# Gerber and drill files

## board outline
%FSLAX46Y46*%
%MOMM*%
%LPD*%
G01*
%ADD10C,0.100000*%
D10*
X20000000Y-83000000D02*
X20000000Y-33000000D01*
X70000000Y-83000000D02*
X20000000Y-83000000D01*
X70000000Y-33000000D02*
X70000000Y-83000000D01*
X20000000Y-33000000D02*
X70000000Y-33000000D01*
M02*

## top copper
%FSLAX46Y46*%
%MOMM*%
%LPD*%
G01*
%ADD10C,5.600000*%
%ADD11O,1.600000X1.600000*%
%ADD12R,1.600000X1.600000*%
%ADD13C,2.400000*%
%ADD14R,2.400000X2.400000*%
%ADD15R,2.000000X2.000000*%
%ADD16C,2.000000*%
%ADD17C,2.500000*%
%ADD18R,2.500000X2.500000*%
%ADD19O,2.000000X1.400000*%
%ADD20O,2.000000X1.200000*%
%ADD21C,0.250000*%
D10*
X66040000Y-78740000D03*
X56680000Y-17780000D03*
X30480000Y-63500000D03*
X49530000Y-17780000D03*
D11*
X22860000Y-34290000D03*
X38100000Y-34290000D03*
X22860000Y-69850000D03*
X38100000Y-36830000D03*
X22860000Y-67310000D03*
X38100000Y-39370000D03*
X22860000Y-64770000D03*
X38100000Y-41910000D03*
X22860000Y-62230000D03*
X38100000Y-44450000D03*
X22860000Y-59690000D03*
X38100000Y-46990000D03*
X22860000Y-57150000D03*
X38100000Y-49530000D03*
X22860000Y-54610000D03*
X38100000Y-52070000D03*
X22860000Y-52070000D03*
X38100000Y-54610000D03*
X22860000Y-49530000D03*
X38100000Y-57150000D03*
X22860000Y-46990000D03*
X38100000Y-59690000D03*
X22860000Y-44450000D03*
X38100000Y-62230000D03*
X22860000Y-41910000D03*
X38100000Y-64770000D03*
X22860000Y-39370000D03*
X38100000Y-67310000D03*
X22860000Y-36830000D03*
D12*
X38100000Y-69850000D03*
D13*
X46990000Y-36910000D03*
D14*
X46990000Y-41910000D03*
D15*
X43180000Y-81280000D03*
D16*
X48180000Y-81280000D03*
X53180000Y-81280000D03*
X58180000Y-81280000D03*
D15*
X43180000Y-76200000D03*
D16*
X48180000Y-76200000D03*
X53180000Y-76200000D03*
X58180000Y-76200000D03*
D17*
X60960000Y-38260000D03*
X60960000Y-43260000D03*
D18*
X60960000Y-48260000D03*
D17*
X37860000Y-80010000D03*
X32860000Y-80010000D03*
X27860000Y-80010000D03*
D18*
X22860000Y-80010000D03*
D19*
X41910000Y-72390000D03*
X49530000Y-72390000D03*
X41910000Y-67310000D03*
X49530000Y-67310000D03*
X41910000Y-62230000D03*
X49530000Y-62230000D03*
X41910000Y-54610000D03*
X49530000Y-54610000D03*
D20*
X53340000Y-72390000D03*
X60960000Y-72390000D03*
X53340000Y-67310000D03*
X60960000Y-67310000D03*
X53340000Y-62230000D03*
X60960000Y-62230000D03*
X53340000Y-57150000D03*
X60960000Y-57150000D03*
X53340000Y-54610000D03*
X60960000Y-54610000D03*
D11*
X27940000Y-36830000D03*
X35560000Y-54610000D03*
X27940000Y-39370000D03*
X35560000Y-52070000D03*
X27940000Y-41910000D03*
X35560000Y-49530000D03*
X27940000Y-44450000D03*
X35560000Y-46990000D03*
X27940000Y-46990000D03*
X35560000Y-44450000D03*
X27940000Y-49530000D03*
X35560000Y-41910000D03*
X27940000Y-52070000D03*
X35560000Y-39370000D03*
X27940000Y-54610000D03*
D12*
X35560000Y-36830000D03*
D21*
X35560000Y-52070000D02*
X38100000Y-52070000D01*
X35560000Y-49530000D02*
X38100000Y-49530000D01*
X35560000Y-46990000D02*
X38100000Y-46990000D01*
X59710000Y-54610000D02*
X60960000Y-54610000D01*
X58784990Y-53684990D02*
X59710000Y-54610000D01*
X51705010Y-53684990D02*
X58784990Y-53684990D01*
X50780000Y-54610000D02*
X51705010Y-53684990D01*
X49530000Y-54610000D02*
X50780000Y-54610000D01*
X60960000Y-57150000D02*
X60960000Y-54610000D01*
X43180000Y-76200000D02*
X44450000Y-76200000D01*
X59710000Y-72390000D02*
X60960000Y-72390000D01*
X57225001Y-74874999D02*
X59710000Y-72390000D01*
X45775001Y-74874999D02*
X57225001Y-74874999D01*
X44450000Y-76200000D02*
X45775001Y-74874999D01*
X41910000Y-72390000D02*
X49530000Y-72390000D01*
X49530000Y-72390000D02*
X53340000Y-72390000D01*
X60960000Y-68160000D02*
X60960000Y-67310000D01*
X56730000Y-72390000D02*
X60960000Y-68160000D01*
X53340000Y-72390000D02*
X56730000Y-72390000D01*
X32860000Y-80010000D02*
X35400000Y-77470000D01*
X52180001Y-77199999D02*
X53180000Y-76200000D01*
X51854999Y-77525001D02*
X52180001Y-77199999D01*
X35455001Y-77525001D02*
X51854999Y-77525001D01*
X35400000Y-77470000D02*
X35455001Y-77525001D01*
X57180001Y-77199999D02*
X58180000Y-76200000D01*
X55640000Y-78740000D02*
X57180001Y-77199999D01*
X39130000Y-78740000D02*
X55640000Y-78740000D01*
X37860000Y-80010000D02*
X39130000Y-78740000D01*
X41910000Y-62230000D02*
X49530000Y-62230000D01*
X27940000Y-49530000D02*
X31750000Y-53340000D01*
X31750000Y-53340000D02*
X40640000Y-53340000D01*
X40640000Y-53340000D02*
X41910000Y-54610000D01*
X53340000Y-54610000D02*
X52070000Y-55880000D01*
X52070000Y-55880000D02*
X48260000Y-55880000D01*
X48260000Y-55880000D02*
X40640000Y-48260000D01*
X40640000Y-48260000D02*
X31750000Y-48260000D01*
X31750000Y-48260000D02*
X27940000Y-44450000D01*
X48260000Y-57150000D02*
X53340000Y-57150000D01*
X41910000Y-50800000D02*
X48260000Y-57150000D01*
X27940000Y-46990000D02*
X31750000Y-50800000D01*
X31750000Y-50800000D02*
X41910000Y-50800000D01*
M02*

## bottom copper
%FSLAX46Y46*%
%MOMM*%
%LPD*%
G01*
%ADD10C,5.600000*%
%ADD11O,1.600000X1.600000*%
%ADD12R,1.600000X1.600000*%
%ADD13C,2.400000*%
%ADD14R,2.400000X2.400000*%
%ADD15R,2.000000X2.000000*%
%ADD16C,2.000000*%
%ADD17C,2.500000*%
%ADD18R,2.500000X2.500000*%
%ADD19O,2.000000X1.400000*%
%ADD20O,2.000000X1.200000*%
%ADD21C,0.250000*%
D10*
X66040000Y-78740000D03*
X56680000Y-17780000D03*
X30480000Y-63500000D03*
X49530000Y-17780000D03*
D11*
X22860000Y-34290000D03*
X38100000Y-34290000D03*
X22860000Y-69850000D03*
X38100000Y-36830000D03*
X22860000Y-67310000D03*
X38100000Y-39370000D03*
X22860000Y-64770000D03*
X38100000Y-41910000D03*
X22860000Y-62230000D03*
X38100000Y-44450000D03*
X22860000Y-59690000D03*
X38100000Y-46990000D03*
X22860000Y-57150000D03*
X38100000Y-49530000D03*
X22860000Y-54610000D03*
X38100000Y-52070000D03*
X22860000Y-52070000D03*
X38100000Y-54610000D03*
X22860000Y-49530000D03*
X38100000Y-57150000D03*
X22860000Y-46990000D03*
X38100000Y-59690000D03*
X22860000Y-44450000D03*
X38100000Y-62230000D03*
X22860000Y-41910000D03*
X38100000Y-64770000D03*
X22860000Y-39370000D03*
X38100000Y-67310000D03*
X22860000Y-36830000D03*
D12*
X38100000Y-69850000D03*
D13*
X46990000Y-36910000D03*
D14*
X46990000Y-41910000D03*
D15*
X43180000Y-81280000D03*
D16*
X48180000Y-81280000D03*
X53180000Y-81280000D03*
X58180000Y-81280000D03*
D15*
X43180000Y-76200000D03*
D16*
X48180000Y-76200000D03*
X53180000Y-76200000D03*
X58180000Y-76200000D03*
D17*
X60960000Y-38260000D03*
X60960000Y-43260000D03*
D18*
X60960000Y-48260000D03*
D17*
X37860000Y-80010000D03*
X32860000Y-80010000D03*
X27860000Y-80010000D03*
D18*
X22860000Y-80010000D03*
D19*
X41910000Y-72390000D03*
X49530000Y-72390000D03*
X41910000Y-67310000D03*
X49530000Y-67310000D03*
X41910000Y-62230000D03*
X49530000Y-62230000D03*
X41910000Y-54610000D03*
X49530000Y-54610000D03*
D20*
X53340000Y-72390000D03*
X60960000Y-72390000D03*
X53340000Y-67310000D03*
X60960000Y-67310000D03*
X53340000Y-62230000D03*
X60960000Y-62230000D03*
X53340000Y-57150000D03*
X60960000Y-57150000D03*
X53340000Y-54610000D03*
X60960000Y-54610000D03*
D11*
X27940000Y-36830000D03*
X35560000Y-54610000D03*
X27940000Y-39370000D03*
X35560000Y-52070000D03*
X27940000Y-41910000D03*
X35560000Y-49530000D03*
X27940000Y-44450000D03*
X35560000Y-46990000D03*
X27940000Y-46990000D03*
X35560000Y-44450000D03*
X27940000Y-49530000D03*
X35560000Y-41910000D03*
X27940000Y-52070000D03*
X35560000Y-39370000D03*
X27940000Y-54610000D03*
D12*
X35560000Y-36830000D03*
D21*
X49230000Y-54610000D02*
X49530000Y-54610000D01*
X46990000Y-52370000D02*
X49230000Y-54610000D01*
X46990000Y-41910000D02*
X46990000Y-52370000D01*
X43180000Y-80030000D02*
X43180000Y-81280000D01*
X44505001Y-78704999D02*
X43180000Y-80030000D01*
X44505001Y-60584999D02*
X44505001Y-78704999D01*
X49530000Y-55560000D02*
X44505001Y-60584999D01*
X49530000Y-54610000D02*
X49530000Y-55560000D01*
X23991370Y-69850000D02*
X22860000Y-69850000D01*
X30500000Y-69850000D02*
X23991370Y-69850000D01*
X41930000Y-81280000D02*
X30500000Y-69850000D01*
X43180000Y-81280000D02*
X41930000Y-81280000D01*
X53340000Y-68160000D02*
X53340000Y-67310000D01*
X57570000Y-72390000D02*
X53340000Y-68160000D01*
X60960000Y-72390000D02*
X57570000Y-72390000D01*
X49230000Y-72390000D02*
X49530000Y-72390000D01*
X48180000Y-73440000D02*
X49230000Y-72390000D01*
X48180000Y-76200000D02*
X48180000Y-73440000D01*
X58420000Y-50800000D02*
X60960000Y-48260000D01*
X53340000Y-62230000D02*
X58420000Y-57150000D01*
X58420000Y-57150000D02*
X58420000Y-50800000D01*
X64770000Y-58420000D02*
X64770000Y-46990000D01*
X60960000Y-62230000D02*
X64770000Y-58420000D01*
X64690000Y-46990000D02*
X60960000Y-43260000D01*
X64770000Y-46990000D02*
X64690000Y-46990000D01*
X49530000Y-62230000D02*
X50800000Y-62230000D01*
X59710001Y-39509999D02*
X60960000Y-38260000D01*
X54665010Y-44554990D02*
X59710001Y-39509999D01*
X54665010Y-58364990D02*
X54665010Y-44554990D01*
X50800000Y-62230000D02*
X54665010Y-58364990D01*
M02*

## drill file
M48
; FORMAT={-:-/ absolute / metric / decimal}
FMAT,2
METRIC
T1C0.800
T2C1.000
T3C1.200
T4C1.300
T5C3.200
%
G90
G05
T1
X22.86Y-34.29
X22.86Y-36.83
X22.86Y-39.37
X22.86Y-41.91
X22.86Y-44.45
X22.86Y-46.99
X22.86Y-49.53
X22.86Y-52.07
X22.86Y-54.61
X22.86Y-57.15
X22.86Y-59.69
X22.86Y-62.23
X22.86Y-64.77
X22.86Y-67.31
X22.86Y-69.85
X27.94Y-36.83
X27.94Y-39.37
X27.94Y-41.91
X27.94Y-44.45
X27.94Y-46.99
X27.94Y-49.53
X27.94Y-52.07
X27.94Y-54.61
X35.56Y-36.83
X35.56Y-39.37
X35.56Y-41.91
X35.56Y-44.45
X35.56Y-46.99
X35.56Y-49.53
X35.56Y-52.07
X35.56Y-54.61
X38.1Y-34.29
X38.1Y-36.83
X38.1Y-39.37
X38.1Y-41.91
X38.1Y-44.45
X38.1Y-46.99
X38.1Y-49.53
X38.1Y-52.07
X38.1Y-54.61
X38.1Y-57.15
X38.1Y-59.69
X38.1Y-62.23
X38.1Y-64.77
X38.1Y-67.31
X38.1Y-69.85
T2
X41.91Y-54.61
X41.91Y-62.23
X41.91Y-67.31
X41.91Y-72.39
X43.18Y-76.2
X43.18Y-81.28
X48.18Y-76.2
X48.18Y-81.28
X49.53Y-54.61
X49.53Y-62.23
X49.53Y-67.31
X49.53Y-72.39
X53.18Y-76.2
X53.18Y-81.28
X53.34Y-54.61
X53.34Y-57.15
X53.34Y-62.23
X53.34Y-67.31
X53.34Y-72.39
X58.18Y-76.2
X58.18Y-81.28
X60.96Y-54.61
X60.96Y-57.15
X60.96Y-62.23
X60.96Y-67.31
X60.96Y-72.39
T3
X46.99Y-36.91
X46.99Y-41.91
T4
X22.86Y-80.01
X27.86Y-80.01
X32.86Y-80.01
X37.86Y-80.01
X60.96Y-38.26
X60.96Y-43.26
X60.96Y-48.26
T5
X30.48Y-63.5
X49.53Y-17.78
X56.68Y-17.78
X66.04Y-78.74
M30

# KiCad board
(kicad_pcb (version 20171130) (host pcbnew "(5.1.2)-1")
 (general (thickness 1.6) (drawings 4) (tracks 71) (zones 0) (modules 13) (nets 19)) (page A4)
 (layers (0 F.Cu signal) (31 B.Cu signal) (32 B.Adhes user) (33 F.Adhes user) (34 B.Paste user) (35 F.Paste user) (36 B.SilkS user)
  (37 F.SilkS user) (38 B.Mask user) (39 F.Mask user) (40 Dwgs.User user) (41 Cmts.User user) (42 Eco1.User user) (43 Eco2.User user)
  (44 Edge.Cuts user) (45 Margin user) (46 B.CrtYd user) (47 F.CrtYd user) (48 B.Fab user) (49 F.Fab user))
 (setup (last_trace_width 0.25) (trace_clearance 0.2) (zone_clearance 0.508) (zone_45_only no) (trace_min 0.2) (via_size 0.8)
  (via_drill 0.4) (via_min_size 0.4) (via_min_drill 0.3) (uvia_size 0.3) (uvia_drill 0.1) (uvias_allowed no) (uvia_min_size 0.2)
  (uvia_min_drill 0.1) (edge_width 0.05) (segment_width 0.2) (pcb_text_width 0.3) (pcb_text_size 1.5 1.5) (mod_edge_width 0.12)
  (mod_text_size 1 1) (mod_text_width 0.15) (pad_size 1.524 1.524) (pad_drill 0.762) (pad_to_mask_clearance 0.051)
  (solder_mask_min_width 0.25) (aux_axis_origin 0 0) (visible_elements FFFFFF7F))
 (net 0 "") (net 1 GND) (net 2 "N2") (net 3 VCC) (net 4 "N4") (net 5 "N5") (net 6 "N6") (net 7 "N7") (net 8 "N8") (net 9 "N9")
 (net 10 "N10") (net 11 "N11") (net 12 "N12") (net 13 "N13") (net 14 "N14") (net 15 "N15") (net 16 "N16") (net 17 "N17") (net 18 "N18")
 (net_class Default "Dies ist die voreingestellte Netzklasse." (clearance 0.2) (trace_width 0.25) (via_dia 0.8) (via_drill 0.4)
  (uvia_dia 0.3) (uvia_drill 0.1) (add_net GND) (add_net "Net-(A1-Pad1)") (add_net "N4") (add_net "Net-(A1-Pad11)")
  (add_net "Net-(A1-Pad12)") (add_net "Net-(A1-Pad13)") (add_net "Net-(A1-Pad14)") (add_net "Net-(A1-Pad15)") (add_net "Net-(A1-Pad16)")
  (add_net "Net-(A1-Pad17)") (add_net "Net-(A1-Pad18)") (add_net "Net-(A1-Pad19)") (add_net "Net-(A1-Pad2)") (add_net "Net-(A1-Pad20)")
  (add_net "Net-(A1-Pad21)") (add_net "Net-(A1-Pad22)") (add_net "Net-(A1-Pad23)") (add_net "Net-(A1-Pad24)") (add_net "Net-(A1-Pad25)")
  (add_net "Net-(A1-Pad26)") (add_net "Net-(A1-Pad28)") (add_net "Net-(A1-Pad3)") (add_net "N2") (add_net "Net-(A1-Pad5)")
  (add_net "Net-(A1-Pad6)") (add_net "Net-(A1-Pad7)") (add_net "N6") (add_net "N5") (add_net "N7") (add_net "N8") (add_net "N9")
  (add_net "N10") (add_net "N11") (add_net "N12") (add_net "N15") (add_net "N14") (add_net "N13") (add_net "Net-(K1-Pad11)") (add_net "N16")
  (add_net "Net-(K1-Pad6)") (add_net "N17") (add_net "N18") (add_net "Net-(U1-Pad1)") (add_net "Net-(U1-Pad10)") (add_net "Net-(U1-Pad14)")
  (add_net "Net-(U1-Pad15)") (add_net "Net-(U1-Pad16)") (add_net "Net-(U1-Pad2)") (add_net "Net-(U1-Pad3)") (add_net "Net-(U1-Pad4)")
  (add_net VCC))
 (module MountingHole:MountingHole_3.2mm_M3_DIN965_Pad (layer F.Cu) (at 66.04 78.74)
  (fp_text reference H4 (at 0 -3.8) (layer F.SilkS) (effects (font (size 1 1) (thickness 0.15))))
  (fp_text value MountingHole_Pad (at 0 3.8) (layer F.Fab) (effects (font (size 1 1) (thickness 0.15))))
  (pad 1 thru_hole circle (at 0 0) (size 5.6 5.6) (drill 3.2) (layers *.Cu *.Mask) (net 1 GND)))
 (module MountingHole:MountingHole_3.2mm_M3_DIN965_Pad (layer F.Cu) (at 56.68 17.78)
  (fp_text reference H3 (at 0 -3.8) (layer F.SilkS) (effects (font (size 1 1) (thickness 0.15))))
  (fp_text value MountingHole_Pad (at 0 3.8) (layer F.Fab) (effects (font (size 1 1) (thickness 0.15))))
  (pad 1 thru_hole circle (at 0 0) (size 5.6 5.6) (drill 3.2) (layers *.Cu *.Mask) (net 1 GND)))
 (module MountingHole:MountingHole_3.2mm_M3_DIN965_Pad (layer F.Cu) (at 30.48 63.5)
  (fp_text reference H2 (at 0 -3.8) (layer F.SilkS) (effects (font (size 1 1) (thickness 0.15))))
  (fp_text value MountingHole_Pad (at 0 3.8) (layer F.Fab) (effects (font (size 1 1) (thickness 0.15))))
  (pad 1 thru_hole circle (at 0 0) (size 5.6 5.6) (drill 3.2) (layers *.Cu *.Mask) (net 1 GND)))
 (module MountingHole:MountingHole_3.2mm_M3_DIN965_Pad (layer F.Cu) (at 49.53 17.78)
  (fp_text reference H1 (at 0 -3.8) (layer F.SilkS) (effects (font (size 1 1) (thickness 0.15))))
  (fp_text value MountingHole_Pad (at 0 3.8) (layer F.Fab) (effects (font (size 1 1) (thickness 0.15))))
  (pad 1 thru_hole circle (at 0 0) (size 5.6 5.6) (drill 3.2) (layers *.Cu *.Mask) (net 1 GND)))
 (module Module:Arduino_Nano (layer F.Cu) (at 38.1 69.85 180)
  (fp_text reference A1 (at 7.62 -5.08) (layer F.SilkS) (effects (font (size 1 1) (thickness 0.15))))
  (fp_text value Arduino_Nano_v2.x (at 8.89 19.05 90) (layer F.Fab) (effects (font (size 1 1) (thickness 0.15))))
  (pad 16 thru_hole oval (at 15.24 35.56 180) (size 1.6 1.6) (drill 0.8) (layers *.Cu *.Mask))
  (pad 15 thru_hole oval (at 0 35.56 180) (size 1.6 1.6) (drill 0.8) (layers *.Cu *.Mask))
  (pad 30 thru_hole oval (at 15.24 0 180) (size 1.6 1.6) (drill 0.8) (layers *.Cu *.Mask) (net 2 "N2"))
  (pad 14 thru_hole oval (at 0 33.02 180) (size 1.6 1.6) (drill 0.8) (layers *.Cu *.Mask))
  (pad 29 thru_hole oval (at 15.24 2.54 180) (size 1.6 1.6) (drill 0.8) (layers *.Cu *.Mask) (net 1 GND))
  (pad 13 thru_hole oval (at 0 30.48 180) (size 1.6 1.6) (drill 0.8) (layers *.Cu *.Mask))
  (pad 28 thru_hole oval (at 15.24 5.08 180) (size 1.6 1.6) (drill 0.8) (layers *.Cu *.Mask))
  (pad 12 thru_hole oval (at 0 27.94 180) (size 1.6 1.6) (drill 0.8) (layers *.Cu *.Mask))
  (pad 27 thru_hole oval (at 15.24 7.62 180) (size 1.6 1.6) (drill 0.8) (layers *.Cu *.Mask) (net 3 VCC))
  (pad 11 thru_hole oval (at 0 25.4 180) (size 1.6 1.6) (drill 0.8) (layers *.Cu *.Mask))
  (pad 26 thru_hole oval (at 15.24 10.16 180) (size 1.6 1.6) (drill 0.8) (layers *.Cu *.Mask))
  (pad 10 thru_hole oval (at 0 22.86 180) (size 1.6 1.6) (drill 0.8) (layers *.Cu *.Mask) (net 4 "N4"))
  (pad 25 thru_hole oval (at 15.24 12.7 180) (size 1.6 1.6) (drill 0.8) (layers *.Cu *.Mask))
  (pad 9 thru_hole oval (at 0 20.32 180) (size 1.6 1.6) (drill 0.8) (layers *.Cu *.Mask) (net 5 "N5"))
  (pad 24 thru_hole oval (at 15.24 15.24 180) (size 1.6 1.6) (drill 0.8) (layers *.Cu *.Mask))
  (pad 8 thru_hole oval (at 0 17.78 180) (size 1.6 1.6) (drill 0.8) (layers *.Cu *.Mask) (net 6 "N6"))
  (pad 23 thru_hole oval (at 15.24 17.78 180) (size 1.6 1.6) (drill 0.8) (layers *.Cu *.Mask))
  (pad 7 thru_hole oval (at 0 15.24 180) (size 1.6 1.6) (drill 0.8) (layers *.Cu *.Mask))
  (pad 22 thru_hole oval (at 15.24 20.32 180) (size 1.6 1.6) (drill 0.8) (layers *.Cu *.Mask))
  (pad 6 thru_hole oval (at 0 12.7 180) (size 1.6 1.6) (drill 0.8) (layers *.Cu *.Mask))
  (pad 21 thru_hole oval (at 15.24 22.86 180) (size 1.6 1.6) (drill 0.8) (layers *.Cu *.Mask))
  (pad 5 thru_hole oval (at 0 10.16 180) (size 1.6 1.6) (drill 0.8) (layers *.Cu *.Mask))
  (pad 20 thru_hole oval (at 15.24 25.4 180) (size 1.6 1.6) (drill 0.8) (layers *.Cu *.Mask))
  (pad 4 thru_hole oval (at 0 7.62 180) (size 1.6 1.6) (drill 0.8) (layers *.Cu *.Mask) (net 1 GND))
  (pad 19 thru_hole oval (at 15.24 27.94 180) (size 1.6 1.6) (drill 0.8) (layers *.Cu *.Mask))
  (pad 3 thru_hole oval (at 0 5.08 180) (size 1.6 1.6) (drill 0.8) (layers *.Cu *.Mask))
  (pad 18 thru_hole oval (at 15.24 30.48 180) (size 1.6 1.6) (drill 0.8) (layers *.Cu *.Mask))
  (pad 2 thru_hole oval (at 0 2.54 180) (size 1.6 1.6) (drill 0.8) (layers *.Cu *.Mask))
  (pad 17 thru_hole oval (at 15.24 33.02 180) (size 1.6 1.6) (drill 0.8) (layers *.Cu *.Mask))
  (pad 1 thru_hole rect (at 0 0 180) (size 1.6 1.6) (drill 0.8) (layers *.Cu *.Mask)))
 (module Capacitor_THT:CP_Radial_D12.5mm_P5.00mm (layer F.Cu) (at 46.99 41.91 90)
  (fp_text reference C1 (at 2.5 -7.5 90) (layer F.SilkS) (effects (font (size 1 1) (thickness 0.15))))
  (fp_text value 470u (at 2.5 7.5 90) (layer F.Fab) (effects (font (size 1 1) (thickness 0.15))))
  (pad 2 thru_hole circle (at 5 0 90) (size 2.4 2.4) (drill 1.2) (layers *.Cu *.Mask) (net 1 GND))
  (pad 1 thru_hole rect (at 0 0 90) (size 2.4 2.4) (drill 1.2) (layers *.Cu *.Mask) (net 3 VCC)))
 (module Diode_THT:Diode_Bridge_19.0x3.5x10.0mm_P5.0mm (layer F.Cu) (at 43.18 81.28)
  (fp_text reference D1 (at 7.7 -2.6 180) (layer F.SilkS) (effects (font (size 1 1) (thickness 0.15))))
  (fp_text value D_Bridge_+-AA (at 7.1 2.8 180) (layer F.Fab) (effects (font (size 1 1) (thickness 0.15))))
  (pad 1 thru_hole rect (at 0 0) (size 2 2) (drill 1) (layers *.Cu *.Mask) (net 2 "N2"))
  (pad 2 thru_hole circle (at 5 0) (size 2 2) (drill 1) (layers *.Cu *.Mask) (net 1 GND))
  (pad 3 thru_hole circle (at 10 0) (size 2 2) (drill 1) (layers *.Cu *.Mask) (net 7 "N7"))
  (pad 4 thru_hole circle (at 15 0) (size 2 2) (drill 1) (layers *.Cu *.Mask) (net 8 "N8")))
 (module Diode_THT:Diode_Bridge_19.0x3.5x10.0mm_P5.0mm (layer F.Cu) (at 43.18 76.2)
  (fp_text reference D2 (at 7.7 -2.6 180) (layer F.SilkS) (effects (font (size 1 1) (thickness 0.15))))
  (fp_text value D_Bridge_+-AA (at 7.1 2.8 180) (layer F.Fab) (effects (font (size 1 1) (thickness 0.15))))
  (pad 1 thru_hole rect (at 0 0) (size 2 2) (drill 1) (layers *.Cu *.Mask) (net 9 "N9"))
  (pad 2 thru_hole circle (at 5 0) (size 2 2) (drill 1) (layers *.Cu *.Mask) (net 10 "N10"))
  (pad 3 thru_hole circle (at 10 0) (size 2 2) (drill 1) (layers *.Cu *.Mask) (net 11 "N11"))
  (pad 4 thru_hole circle (at 15 0) (size 2 2) (drill 1) (layers *.Cu *.Mask) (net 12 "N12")))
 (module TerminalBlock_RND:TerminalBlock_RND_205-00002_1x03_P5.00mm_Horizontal (layer F.Cu) (at 60.96 48.26 90)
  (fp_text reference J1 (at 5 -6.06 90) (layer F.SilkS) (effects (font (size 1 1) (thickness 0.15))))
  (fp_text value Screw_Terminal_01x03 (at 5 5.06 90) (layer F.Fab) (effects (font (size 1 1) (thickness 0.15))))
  (pad 3 thru_hole circle (at 10 0 90) (size 2.5 2.5) (drill 1.3) (layers *.Cu *.Mask) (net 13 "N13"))
  (pad 2 thru_hole circle (at 5 0 90) (size 2.5 2.5) (drill 1.3) (layers *.Cu *.Mask) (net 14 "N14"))
  (pad 1 thru_hole rect (at 0 0 90) (size 2.5 2.5) (drill 1.3) (layers *.Cu *.Mask) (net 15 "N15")))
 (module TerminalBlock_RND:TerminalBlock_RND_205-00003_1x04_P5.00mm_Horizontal (layer F.Cu) (at 22.86 80.01)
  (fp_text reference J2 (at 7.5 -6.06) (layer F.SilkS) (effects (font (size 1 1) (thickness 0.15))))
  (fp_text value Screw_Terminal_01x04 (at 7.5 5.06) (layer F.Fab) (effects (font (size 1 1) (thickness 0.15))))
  (pad 4 thru_hole circle (at 15 0) (size 2.5 2.5) (drill 1.3) (layers *.Cu *.Mask) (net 12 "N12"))
  (pad 3 thru_hole circle (at 10 0) (size 2.5 2.5) (drill 1.3) (layers *.Cu *.Mask) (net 11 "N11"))
  (pad 2 thru_hole circle (at 5 0) (size 2.5 2.5) (drill 1.3) (layers *.Cu *.Mask) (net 8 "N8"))
  (pad 1 thru_hole rect (at 0 0) (size 2.5 2.5) (drill 1.3) (layers *.Cu *.Mask) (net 7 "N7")))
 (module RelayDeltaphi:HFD (layer F.Cu) (at 45.72 63.5 270)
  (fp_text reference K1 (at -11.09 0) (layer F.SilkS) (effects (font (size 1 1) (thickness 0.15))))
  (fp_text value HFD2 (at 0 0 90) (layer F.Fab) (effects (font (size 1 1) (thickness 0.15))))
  (pad 9 thru_hole oval (at 8.89 3.81 270) (size 1.4 2) (drill 1) (layers *.Cu *.Mask) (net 10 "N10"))
  (pad 8 thru_hole oval (at 8.89 -3.81 270) (size 1.4 2) (drill 1) (layers *.Cu *.Mask) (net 10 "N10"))
  (pad 11 thru_hole oval (at 3.81 3.81 270) (size 1.4 2) (drill 1) (layers *.Cu *.Mask))
  (pad 6 thru_hole oval (at 3.81 -3.81 270) (size 1.4 2) (drill 1) (layers *.Cu *.Mask))
  (pad 13 thru_hole oval (at -1.27 3.81 270) (size 1.4 2) (drill 1) (layers *.Cu *.Mask) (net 13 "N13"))
  (pad 4 thru_hole oval (at -1.27 -3.81 270) (size 1.4 2) (drill 1) (layers *.Cu *.Mask) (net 13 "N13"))
  (pad 16 thru_hole oval (at -8.89 3.81 270) (size 1.4 2) (drill 1) (layers *.Cu *.Mask) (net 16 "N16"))
  (pad 1 thru_hole oval (at -8.89 -3.81 270) (size 1.4 2) (drill 1) (layers *.Cu *.Mask) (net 3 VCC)))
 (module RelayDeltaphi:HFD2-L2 (layer F.Cu) (at 57.15 63.5 270)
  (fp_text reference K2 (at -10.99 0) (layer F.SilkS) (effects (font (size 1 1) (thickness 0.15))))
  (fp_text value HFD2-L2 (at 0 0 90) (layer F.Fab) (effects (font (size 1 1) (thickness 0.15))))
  (pad 9 thru_hole oval (at 8.89 3.81 270) (size 1.2 2) (drill 1) (layers *.Cu *.Mask) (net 10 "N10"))
  (pad 8 thru_hole oval (at 8.89 -3.81 270) (size 1.2 2) (drill 1) (layers *.Cu *.Mask) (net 9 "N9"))
  (pad 11 thru_hole oval (at 3.81 3.81 270) (size 1.2 2) (drill 1) (layers *.Cu *.Mask) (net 9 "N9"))
  (pad 6 thru_hole oval (at 3.81 -3.81 270) (size 1.2 2) (drill 1) (layers *.Cu *.Mask) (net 10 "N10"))
  (pad 13 thru_hole oval (at -1.27 3.81 270) (size 1.2 2) (drill 1) (layers *.Cu *.Mask) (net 15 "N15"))
  (pad 4 thru_hole oval (at -1.27 -3.81 270) (size 1.2 2) (drill 1) (layers *.Cu *.Mask) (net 14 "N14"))
  (pad 15 thru_hole oval (at -6.35 3.81 270) (size 1.2 2) (drill 1) (layers *.Cu *.Mask) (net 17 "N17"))
  (pad 2 thru_hole oval (at -6.35 -3.81 270) (size 1.2 2) (drill 1) (layers *.Cu *.Mask) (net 3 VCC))
  (pad 16 thru_hole oval (at -8.89 3.81 270) (size 1.2 2) (drill 1) (layers *.Cu *.Mask) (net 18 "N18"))
  (pad 1 thru_hole oval (at -8.89 -3.81 270) (size 1.2 2) (drill 1) (layers *.Cu *.Mask) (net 3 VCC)))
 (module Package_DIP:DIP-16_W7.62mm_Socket (layer B.Cu) (at 35.56 36.83 180)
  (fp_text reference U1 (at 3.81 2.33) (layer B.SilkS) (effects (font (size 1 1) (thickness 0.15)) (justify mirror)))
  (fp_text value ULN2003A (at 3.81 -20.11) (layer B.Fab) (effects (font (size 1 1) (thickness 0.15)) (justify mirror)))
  (pad 16 thru_hole oval (at 7.62 0 180) (size 1.6 1.6) (drill 0.8) (layers *.Cu *.Mask))
  (pad 8 thru_hole oval (at 0 -17.78 180) (size 1.6 1.6) (drill 0.8) (layers *.Cu *.Mask) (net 1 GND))
  (pad 15 thru_hole oval (at 7.62 -2.54 180) (size 1.6 1.6) (drill 0.8) (layers *.Cu *.Mask))
  (pad 7 thru_hole oval (at 0 -15.24 180) (size 1.6 1.6) (drill 0.8) (layers *.Cu *.Mask) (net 6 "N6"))
  (pad 14 thru_hole oval (at 7.62 -5.08 180) (size 1.6 1.6) (drill 0.8) (layers *.Cu *.Mask))
  (pad 6 thru_hole oval (at 0 -12.7 180) (size 1.6 1.6) (drill 0.8) (layers *.Cu *.Mask) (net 5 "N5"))
  (pad 13 thru_hole oval (at 7.62 -7.62 180) (size 1.6 1.6) (drill 0.8) (layers *.Cu *.Mask) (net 18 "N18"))
  (pad 5 thru_hole oval (at 0 -10.16 180) (size 1.6 1.6) (drill 0.8) (layers *.Cu *.Mask) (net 4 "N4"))
  (pad 12 thru_hole oval (at 7.62 -10.16 180) (size 1.6 1.6) (drill 0.8) (layers *.Cu *.Mask) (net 17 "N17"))
  (pad 4 thru_hole oval (at 0 -7.62 180) (size 1.6 1.6) (drill 0.8) (layers *.Cu *.Mask))
  (pad 11 thru_hole oval (at 7.62 -12.7 180) (size 1.6 1.6) (drill 0.8) (layers *.Cu *.Mask) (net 16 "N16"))
  (pad 3 thru_hole oval (at 0 -5.08 180) (size 1.6 1.6) (drill 0.8) (layers *.Cu *.Mask))
  (pad 10 thru_hole oval (at 7.62 -15.24 180) (size 1.6 1.6) (drill 0.8) (layers *.Cu *.Mask))
  (pad 2 thru_hole oval (at 0 -2.54 180) (size 1.6 1.6) (drill 0.8) (layers *.Cu *.Mask))
  (pad 9 thru_hole oval (at 7.62 -17.78 180) (size 1.6 1.6) (drill 0.8) (layers *.Cu *.Mask) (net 1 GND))
  (pad 1 thru_hole rect (at 0 0 180) (size 1.6 1.6) (drill 0.8) (layers *.Cu *.Mask)))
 (gr_line (start 20 83) (end 20 33) (layer Edge.Cuts) (width 0.1))
 (gr_line (start 70 83) (end 20 83) (layer Edge.Cuts) (width 0.1))
 (gr_line (start 70 33) (end 70 83) (layer Edge.Cuts) (width 0.1))
 (gr_line (start 20 33) (end 70 33) (layer Edge.Cuts) (width 0.1))
 (segment (start 35.56 52.07) (end 38.1 52.07) (width 0.25) (layer F.Cu) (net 6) (status 30))
 (segment (start 35.56 49.53) (end 38.1 49.53) (width 0.25) (layer F.Cu) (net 5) (status 30))
 (segment (start 35.56 46.99) (end 38.1 46.99) (width 0.25) (layer F.Cu) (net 4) (status 30))
 (segment (start 59.71 54.61) (end 60.96 54.61) (width 0.25) (layer F.Cu) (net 3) (status 20))
 (segment (start 58.78499 53.68499) (end 59.71 54.61) (width 0.25) (layer F.Cu) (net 3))
 (segment (start 51.70501 53.68499) (end 58.78499 53.68499) (width 0.25) (layer F.Cu) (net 3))
 (segment (start 50.78 54.61) (end 51.70501 53.68499) (width 0.25) (layer F.Cu) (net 3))
 (segment (start 49.53 54.61) (end 50.78 54.61) (width 0.25) (layer F.Cu) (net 3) (status 10))
 (segment (start 60.96 57.15) (end 60.96 54.61) (width 0.25) (layer F.Cu) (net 3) (status 30))
 (segment (start 49.23 54.61) (end 49.53 54.61) (width 0.25) (layer B.Cu) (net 3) (status 30))
 (segment (start 46.99 52.37) (end 49.23 54.61) (width 0.25) (layer B.Cu) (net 3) (status 20))
 (segment (start 46.99 41.91) (end 46.99 52.37) (width 0.25) (layer B.Cu) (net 3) (status 10))
 (segment (start 43.18 80.03) (end 43.18 81.28) (width 0.25) (layer B.Cu) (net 3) (status 20))
 (segment (start 44.505001 78.704999) (end 43.18 80.03) (width 0.25) (layer B.Cu) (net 3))
 (segment (start 44.505001 60.584999) (end 44.505001 78.704999) (width 0.25) (layer B.Cu) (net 3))
 (segment (start 49.53 55.56) (end 44.505001 60.584999) (width 0.25) (layer B.Cu) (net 3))
 (segment (start 49.53 54.61) (end 49.53 55.56) (width 0.25) (layer B.Cu) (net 3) (status 10))
 (segment (start 23.99137 69.85) (end 22.86 69.85) (width 0.25) (layer B.Cu) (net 3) (status 20))
 (segment (start 30.5 69.85) (end 23.99137 69.85) (width 0.25) (layer B.Cu) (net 3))
 (segment (start 41.93 81.28) (end 30.5 69.85) (width 0.25) (layer B.Cu) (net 3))
 (segment (start 43.18 81.28) (end 41.93 81.28) (width 0.25) (layer B.Cu) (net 3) (status 10))
 (segment (start 53.34 68.16) (end 53.34 67.31) (width 0.25) (layer B.Cu) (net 9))
 (segment (start 57.57 72.39) (end 53.34 68.16) (width 0.25) (layer B.Cu) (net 9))
 (segment (start 60.96 72.39) (end 57.57 72.39) (width 0.25) (layer B.Cu) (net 9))
 (segment (start 43.18 76.2) (end 44.45 76.2) (width 0.25) (layer F.Cu) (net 9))
 (segment (start 59.71 72.39) (end 60.96 72.39) (width 0.25) (layer F.Cu) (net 9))
 (segment (start 57.225001 74.874999) (end 59.71 72.39) (width 0.25) (layer F.Cu) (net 9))
 (segment (start 45.775001 74.874999) (end 57.225001 74.874999) (width 0.25) (layer F.Cu) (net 9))
 (segment (start 44.45 76.2) (end 45.775001 74.874999) (width 0.25) (layer F.Cu) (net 9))
 (segment (start 41.91 72.39) (end 49.53 72.39) (width 0.25) (layer F.Cu) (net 10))
 (segment (start 49.53 72.39) (end 53.34 72.39) (width 0.25) (layer F.Cu) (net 10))
 (segment (start 60.96 68.16) (end 60.96 67.31) (width 0.25) (layer F.Cu) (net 10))
 (segment (start 56.73 72.39) (end 60.96 68.16) (width 0.25) (layer F.Cu) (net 10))
 (segment (start 53.34 72.39) (end 56.73 72.39) (width 0.25) (layer F.Cu) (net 10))
 (segment (start 49.23 72.39) (end 49.53 72.39) (width 0.25) (layer B.Cu) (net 10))
 (segment (start 48.18 73.44) (end 49.23 72.39) (width 0.25) (layer B.Cu) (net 10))
 (segment (start 48.18 76.2) (end 48.18 73.44) (width 0.25) (layer B.Cu) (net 10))
 (segment (start 32.86 80.01) (end 35.4 77.47) (width 0.25) (layer F.Cu) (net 11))
 (segment (start 52.180001 77.199999) (end 53.18 76.2) (width 0.25) (layer F.Cu) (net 11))
 (segment (start 51.854999 77.525001) (end 52.180001 77.199999) (width 0.25) (layer F.Cu) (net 11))
 (segment (start 35.455001 77.525001) (end 51.854999 77.525001) (width 0.25) (layer F.Cu) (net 11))
 (segment (start 35.4 77.47) (end 35.455001 77.525001) (width 0.25) (layer F.Cu) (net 11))
 (segment (start 57.180001 77.199999) (end 58.18 76.2) (width 0.25) (layer F.Cu) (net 12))
 (segment (start 55.64 78.74) (end 57.180001 77.199999) (width 0.25) (layer F.Cu) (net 12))
 (segment (start 39.13 78.74) (end 55.64 78.74) (width 0.25) (layer F.Cu) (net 12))
 (segment (start 37.86 80.01) (end 39.13 78.74) (width 0.25) (layer F.Cu) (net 12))
 (segment (start 58.42 50.8) (end 60.96 48.26) (width 0.25) (layer B.Cu) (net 15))
 (segment (start 53.34 62.23) (end 58.42 57.15) (width 0.25) (layer B.Cu) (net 15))
 (segment (start 58.42 57.15) (end 58.42 50.8) (width 0.25) (layer B.Cu) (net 15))
 (segment (start 64.77 58.42) (end 64.77 46.99) (width 0.25) (layer B.Cu) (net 14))
 (segment (start 60.96 62.23) (end 64.77 58.42) (width 0.25) (layer B.Cu) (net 14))
 (segment (start 64.69 46.99) (end 60.96 43.26) (width 0.25) (layer B.Cu) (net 14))
 (segment (start 64.77 46.99) (end 64.69 46.99) (width 0.25) (layer B.Cu) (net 14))
 (segment (start 49.53 62.23) (end 50.8 62.23) (width 0.25) (layer B.Cu) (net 13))
 (segment (start 59.710001 39.509999) (end 60.96 38.26) (width 0.25) (layer B.Cu) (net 13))
 (segment (start 54.66501 44.55499) (end 59.710001 39.509999) (width 0.25) (layer B.Cu) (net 13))
 (segment (start 54.66501 58.36499) (end 54.66501 44.55499) (width 0.25) (layer B.Cu) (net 13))
 (segment (start 50.8 62.23) (end 54.66501 58.36499) (width 0.25) (layer B.Cu) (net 13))
 (segment (start 41.91 62.23) (end 49.53 62.23) (width 0.25) (layer F.Cu) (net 13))
 (segment (start 27.94 49.53) (end 31.75 53.34) (width 0.25) (layer F.Cu) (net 16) (status 10))
 (segment (start 31.75 53.34) (end 40.64 53.34) (width 0.25) (layer F.Cu) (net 16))
 (segment (start 40.64 53.34) (end 41.91 54.61) (width 0.25) (layer F.Cu) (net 16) (status 20))
 (segment (start 53.34 54.61) (end 52.07 55.88) (width 0.25) (layer F.Cu) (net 18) (status 10))
 (segment (start 52.07 55.88) (end 48.26 55.88) (width 0.25) (layer F.Cu) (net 18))
 (segment (start 48.26 55.88) (end 40.64 48.26) (width 0.25) (layer F.Cu) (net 18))
 (segment (start 40.64 48.26) (end 31.75 48.26) (width 0.25) (layer F.Cu) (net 18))
 (segment (start 31.75 48.26) (end 27.94 44.45) (width 0.25) (layer F.Cu) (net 18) (status 20))
 (segment (start 48.26 57.15) (end 53.34 57.15) (width 0.25) (layer F.Cu) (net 17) (status 20))
 (segment (start 41.91 50.8) (end 48.26 57.15) (width 0.25) (layer F.Cu) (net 17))
 (segment (start 27.94 46.99) (end 31.75 50.8) (width 0.25) (layer F.Cu) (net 17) (status 10))
 (segment (start 31.75 50.8) (end 41.91 50.8) (width 0.25) (layer F.Cu) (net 17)))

